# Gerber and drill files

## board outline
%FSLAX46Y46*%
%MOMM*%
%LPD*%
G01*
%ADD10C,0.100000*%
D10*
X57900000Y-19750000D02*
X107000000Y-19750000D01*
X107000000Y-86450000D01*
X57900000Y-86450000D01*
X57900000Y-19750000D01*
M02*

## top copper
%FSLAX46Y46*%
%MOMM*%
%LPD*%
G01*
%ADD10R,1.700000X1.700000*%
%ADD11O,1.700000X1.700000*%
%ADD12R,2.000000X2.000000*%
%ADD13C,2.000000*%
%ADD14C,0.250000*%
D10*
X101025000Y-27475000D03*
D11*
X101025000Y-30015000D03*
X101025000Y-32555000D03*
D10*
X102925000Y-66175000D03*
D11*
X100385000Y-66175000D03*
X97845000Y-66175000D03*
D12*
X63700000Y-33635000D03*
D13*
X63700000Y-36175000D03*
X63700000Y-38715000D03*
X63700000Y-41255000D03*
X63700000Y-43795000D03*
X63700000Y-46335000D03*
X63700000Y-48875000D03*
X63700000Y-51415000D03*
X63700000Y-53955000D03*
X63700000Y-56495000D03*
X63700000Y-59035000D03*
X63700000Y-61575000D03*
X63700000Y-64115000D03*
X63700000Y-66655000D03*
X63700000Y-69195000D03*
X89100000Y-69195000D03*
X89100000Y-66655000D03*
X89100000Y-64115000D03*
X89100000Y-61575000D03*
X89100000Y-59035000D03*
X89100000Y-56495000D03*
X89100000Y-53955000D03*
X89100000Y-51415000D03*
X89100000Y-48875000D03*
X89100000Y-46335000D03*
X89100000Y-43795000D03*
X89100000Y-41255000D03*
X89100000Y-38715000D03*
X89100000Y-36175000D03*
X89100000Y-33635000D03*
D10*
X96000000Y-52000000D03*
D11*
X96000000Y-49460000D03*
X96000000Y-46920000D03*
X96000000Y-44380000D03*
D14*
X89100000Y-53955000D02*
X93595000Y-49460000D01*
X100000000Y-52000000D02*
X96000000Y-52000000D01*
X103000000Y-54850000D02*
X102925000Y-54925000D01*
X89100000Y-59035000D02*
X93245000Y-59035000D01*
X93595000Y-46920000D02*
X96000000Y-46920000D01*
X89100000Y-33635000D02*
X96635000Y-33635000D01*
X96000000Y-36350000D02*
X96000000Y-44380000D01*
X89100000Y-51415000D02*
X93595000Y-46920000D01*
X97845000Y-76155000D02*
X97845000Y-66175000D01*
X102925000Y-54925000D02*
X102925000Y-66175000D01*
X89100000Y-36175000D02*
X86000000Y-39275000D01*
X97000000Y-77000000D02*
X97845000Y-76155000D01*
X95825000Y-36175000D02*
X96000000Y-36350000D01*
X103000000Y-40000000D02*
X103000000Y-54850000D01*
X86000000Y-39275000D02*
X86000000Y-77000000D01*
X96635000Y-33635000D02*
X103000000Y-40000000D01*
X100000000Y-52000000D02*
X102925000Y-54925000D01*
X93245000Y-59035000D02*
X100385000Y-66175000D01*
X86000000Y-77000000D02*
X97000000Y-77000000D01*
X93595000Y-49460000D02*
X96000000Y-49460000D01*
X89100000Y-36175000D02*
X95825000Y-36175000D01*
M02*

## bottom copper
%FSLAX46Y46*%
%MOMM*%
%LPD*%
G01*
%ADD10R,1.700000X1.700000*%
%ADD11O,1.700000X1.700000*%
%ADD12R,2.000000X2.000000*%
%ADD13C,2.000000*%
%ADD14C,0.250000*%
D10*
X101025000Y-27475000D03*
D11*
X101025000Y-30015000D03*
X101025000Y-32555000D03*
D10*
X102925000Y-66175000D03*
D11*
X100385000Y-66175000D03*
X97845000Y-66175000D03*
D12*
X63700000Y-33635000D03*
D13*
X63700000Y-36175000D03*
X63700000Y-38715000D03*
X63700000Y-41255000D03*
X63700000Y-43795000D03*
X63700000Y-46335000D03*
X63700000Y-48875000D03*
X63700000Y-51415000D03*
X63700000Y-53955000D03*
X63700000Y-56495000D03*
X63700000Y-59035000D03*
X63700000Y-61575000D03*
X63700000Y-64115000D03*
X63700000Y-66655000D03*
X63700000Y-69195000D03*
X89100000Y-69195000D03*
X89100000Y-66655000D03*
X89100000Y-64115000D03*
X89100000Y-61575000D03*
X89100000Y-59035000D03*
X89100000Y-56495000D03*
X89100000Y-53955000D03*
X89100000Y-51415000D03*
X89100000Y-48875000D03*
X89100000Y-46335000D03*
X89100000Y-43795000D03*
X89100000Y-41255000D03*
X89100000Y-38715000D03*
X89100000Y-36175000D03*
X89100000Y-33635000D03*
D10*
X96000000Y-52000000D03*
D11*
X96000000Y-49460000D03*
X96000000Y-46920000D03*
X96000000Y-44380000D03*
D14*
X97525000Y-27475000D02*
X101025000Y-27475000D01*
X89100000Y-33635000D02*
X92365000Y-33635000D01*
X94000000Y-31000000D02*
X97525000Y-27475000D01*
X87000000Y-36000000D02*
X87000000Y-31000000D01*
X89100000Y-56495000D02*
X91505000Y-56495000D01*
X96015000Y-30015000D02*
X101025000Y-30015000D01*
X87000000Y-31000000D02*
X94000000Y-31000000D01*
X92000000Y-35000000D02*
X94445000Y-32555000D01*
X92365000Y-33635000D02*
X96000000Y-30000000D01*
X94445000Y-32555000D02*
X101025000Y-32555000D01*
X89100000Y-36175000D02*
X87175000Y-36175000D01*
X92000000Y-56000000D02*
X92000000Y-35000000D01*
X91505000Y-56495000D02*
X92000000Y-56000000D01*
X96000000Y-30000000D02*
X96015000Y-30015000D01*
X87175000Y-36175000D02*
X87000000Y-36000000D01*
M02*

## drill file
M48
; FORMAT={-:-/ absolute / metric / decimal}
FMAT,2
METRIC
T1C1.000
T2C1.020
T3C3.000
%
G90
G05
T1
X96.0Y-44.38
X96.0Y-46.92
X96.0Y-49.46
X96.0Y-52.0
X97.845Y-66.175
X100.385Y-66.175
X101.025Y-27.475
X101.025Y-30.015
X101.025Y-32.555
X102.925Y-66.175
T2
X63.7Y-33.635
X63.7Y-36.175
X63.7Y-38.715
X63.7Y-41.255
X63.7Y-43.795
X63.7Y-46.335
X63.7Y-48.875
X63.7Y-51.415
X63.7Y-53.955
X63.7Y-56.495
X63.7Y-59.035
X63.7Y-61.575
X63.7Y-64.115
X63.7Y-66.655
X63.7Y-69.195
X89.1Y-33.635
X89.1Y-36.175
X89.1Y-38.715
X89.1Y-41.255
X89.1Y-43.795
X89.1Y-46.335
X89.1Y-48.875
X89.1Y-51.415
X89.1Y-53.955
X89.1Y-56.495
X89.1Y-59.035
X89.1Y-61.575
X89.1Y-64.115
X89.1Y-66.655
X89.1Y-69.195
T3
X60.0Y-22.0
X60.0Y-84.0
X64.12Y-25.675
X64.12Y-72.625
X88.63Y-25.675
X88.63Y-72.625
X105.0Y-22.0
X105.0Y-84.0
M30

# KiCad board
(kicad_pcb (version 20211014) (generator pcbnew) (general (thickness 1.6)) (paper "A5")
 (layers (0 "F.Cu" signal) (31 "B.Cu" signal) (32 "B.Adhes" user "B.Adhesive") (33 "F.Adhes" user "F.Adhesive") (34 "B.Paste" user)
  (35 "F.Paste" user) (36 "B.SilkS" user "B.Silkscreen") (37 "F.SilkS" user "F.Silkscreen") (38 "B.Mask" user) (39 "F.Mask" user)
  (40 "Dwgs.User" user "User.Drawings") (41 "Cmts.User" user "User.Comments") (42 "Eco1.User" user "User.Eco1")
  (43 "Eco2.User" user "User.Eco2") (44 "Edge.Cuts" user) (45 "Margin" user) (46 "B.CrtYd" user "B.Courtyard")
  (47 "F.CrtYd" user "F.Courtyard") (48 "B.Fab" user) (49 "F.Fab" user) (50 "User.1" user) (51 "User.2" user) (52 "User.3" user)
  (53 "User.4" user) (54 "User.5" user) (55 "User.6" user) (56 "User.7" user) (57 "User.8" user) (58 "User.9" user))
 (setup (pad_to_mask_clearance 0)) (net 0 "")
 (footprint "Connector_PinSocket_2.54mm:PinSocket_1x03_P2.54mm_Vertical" (layer "F.Cu") (at 101.025 27.475)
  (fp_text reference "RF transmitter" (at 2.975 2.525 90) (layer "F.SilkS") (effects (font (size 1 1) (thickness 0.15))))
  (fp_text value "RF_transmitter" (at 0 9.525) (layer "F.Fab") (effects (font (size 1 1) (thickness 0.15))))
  (pad "1" thru_hole rect (at 0 0) (size 1.7 1.7) (drill 1) (layers *.Cu *.Mask))
  (pad "2" thru_hole oval (at 0 2.54) (size 1.7 1.7) (drill 1) (layers *.Cu *.Mask))
  (pad "3" thru_hole oval (at 0 5.08) (size 1.7 1.7) (drill 1) (layers *.Cu *.Mask)))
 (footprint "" (layer "F.Cu") (at 105 22)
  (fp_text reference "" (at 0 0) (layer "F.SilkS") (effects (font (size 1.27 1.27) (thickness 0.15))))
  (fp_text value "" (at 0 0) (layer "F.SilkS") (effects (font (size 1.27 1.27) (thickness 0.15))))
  (pad "" np_thru_hole circle (at 0 0) (size 3 3) (drill 3) (layers *.Cu *.Mask)))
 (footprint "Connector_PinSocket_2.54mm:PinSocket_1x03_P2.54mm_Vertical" (layer "F.Cu") (at 102.925 66.175 -90)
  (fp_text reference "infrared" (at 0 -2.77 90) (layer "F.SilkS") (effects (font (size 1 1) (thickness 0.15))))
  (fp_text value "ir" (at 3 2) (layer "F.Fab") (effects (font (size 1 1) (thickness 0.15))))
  (pad "1" thru_hole rect (at 0 0 270) (size 1.7 1.7) (drill 1) (layers *.Cu *.Mask))
  (pad "2" thru_hole oval (at 0 2.54 270) (size 1.7 1.7) (drill 1) (layers *.Cu *.Mask))
  (pad "3" thru_hole oval (at 0 5.08 270) (size 1.7 1.7) (drill 1) (layers *.Cu *.Mask)))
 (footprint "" (layer "F.Cu") (at 105 84)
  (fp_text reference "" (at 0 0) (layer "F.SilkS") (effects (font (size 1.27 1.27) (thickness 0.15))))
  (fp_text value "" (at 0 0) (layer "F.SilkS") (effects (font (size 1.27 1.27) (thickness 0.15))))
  (pad "" np_thru_hole circle (at 0 0) (size 3 3) (drill 3) (layers *.Cu *.Mask)))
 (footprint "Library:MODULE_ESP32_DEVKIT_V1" (layer "F.Cu") (at 76.4 49.15)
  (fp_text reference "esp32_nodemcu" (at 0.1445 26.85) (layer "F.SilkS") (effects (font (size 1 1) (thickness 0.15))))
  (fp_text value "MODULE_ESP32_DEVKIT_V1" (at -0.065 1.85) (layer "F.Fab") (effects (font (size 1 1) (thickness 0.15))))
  (pad "" np_thru_hole circle (at -12.28 -23.475) (size 3 3) (drill 3) (layers *.Cu *.Mask))
  (pad "" np_thru_hole circle (at 12.23 23.475) (size 3 3) (drill 3) (layers *.Cu *.Mask))
  (pad "" np_thru_hole circle (at 12.23 -23.475) (size 3 3) (drill 3) (layers *.Cu *.Mask))
  (pad "" np_thru_hole circle (at -12.28 23.475) (size 3 3) (drill 3) (layers *.Cu *.Mask))
  (pad "1" thru_hole rect (at -12.7 -15.515) (size 2 2) (drill 1.02) (layers *.Cu *.Mask))
  (pad "2" thru_hole circle (at -12.7 -12.975) (size 2 2) (drill 1.02) (layers *.Cu *.Mask))
  (pad "3" thru_hole circle (at -12.7 -10.435) (size 2 2) (drill 1.02) (layers *.Cu *.Mask))
  (pad "4" thru_hole circle (at -12.7 -7.895) (size 2 2) (drill 1.02) (layers *.Cu *.Mask))
  (pad "5" thru_hole circle (at -12.7 -5.355) (size 2 2) (drill 1.02) (layers *.Cu *.Mask))
  (pad "6" thru_hole circle (at -12.7 -2.815) (size 2 2) (drill 1.02) (layers *.Cu *.Mask))
  (pad "7" thru_hole circle (at -12.7 -0.275) (size 2 2) (drill 1.02) (layers *.Cu *.Mask))
  (pad "8" thru_hole circle (at -12.7 2.265) (size 2 2) (drill 1.02) (layers *.Cu *.Mask))
  (pad "9" thru_hole circle (at -12.7 4.805) (size 2 2) (drill 1.02) (layers *.Cu *.Mask))
  (pad "10" thru_hole circle (at -12.7 7.345) (size 2 2) (drill 1.02) (layers *.Cu *.Mask))
  (pad "11" thru_hole circle (at -12.7 9.885) (size 2 2) (drill 1.02) (layers *.Cu *.Mask))
  (pad "12" thru_hole circle (at -12.7 12.425) (size 2 2) (drill 1.02) (layers *.Cu *.Mask))
  (pad "13" thru_hole circle (at -12.7 14.965) (size 2 2) (drill 1.02) (layers *.Cu *.Mask))
  (pad "14" thru_hole circle (at -12.7 17.505) (size 2 2) (drill 1.02) (layers *.Cu *.Mask))
  (pad "15" thru_hole circle (at -12.7 20.045) (size 2 2) (drill 1.02) (layers *.Cu *.Mask))
  (pad "16" thru_hole circle (at 12.7 20.045) (size 2 2) (drill 1.02) (layers *.Cu *.Mask))
  (pad "17" thru_hole circle (at 12.7 17.505) (size 2 2) (drill 1.02) (layers *.Cu *.Mask))
  (pad "18" thru_hole circle (at 12.7 14.965) (size 2 2) (drill 1.02) (layers *.Cu *.Mask))
  (pad "19" thru_hole circle (at 12.7 12.425) (size 2 2) (drill 1.02) (layers *.Cu *.Mask))
  (pad "20" thru_hole circle (at 12.7 9.885) (size 2 2) (drill 1.02) (layers *.Cu *.Mask))
  (pad "21" thru_hole circle (at 12.7 7.345) (size 2 2) (drill 1.02) (layers *.Cu *.Mask))
  (pad "22" thru_hole circle (at 12.7 4.805) (size 2 2) (drill 1.02) (layers *.Cu *.Mask))
  (pad "23" thru_hole circle (at 12.7 2.265) (size 2 2) (drill 1.02) (layers *.Cu *.Mask))
  (pad "24" thru_hole circle (at 12.7 -0.275) (size 2 2) (drill 1.02) (layers *.Cu *.Mask))
  (pad "25" thru_hole circle (at 12.7 -2.815) (size 2 2) (drill 1.02) (layers *.Cu *.Mask))
  (pad "26" thru_hole circle (at 12.7 -5.355) (size 2 2) (drill 1.02) (layers *.Cu *.Mask))
  (pad "27" thru_hole circle (at 12.7 -7.895) (size 2 2) (drill 1.02) (layers *.Cu *.Mask))
  (pad "28" thru_hole circle (at 12.7 -10.435) (size 2 2) (drill 1.02) (layers *.Cu *.Mask))
  (pad "29" thru_hole circle (at 12.7 -12.975) (size 2 2) (drill 1.02) (layers *.Cu *.Mask))
  (pad "30" thru_hole circle (at 12.7 -15.515) (size 2 2) (drill 1.02) (layers *.Cu *.Mask))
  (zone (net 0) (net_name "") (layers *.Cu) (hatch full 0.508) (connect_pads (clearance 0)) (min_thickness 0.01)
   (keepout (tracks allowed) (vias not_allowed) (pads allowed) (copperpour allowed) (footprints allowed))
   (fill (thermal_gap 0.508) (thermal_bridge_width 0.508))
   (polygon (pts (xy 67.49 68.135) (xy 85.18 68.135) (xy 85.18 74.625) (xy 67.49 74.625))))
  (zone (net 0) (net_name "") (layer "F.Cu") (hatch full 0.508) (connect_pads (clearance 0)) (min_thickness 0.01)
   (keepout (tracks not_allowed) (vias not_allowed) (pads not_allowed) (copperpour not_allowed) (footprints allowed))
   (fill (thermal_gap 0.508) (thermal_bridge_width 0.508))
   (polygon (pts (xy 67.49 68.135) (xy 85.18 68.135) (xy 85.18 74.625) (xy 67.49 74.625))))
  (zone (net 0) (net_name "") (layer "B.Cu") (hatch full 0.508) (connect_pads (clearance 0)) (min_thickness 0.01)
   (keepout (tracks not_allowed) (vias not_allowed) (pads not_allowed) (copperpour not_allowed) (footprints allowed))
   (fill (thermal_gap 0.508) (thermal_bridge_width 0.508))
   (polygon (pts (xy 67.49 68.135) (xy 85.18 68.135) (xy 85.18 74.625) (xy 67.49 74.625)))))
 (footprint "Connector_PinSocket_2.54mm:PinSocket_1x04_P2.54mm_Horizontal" (layer "F.Cu") (at 96 52 180)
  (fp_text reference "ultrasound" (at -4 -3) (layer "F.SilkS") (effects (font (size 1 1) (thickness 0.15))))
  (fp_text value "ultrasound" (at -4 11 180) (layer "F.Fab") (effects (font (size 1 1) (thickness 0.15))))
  (pad "1" thru_hole rect (at 0 0 180) (size 1.7 1.7) (drill 1) (layers *.Cu *.Mask))
  (pad "2" thru_hole oval (at 0 2.54 180) (size 1.7 1.7) (drill 1) (layers *.Cu *.Mask))
  (pad "3" thru_hole oval (at 0 5.08 180) (size 1.7 1.7) (drill 1) (layers *.Cu *.Mask))
  (pad "4" thru_hole oval (at 0 7.62 180) (size 1.7 1.7) (drill 1) (layers *.Cu *.Mask)))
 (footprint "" (layer "F.Cu") (at 60 22)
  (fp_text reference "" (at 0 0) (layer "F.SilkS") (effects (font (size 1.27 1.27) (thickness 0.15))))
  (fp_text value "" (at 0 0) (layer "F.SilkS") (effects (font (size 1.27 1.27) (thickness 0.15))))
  (pad "" np_thru_hole circle (at 0 0) (size 3 3) (drill 3) (layers *.Cu *.Mask)))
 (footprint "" (layer "F.Cu") (at 60 84)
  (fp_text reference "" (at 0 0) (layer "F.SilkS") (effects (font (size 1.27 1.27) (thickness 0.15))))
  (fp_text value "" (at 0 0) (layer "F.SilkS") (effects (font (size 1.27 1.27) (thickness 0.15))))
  (pad "" np_thru_hole circle (at 0 0) (size 3 3) (drill 3) (layers *.Cu *.Mask)))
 (gr_rect (start 107 19.75) (end 57.9 86.45) (layer "Edge.Cuts") (width 0.1) (fill none))
 (segment (start 89.1 53.955) (end 93.595 49.46) (width 0.25) (layer "F.Cu") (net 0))
 (segment (start 100 52) (end 96 52) (width 0.25) (layer "F.Cu") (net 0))
 (segment (start 103 54.85) (end 102.925 54.925) (width 0.25) (layer "F.Cu") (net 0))
 (segment (start 89.1 59.035) (end 93.245 59.035) (width 0.25) (layer "F.Cu") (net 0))
 (segment (start 93.595 46.92) (end 96 46.92) (width 0.25) (layer "F.Cu") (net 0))
 (segment (start 89.1 33.635) (end 96.635 33.635) (width 0.25) (layer "F.Cu") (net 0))
 (segment (start 96 36.35) (end 96 44.38) (width 0.25) (layer "F.Cu") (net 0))
 (segment (start 89.1 51.415) (end 93.595 46.92) (width 0.25) (layer "F.Cu") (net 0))
 (segment (start 97.845 76.155) (end 97.845 66.175) (width 0.25) (layer "F.Cu") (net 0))
 (segment (start 102.925 54.925) (end 102.925 66.175) (width 0.25) (layer "F.Cu") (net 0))
 (segment (start 89.1 36.175) (end 86 39.275) (width 0.25) (layer "F.Cu") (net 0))
 (segment (start 97 77) (end 97.845 76.155) (width 0.25) (layer "F.Cu") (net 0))
 (segment (start 95.825 36.175) (end 96 36.35) (width 0.25) (layer "F.Cu") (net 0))
 (segment (start 103 40) (end 103 54.85) (width 0.25) (layer "F.Cu") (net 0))
 (segment (start 86 39.275) (end 86 77) (width 0.25) (layer "F.Cu") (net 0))
 (segment (start 96.635 33.635) (end 103 40) (width 0.25) (layer "F.Cu") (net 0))
 (segment (start 100 52) (end 102.925 54.925) (width 0.25) (layer "F.Cu") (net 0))
 (segment (start 93.245 59.035) (end 100.385 66.175) (width 0.25) (layer "F.Cu") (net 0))
 (segment (start 86 77) (end 97 77) (width 0.25) (layer "F.Cu") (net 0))
 (segment (start 93.595 49.46) (end 96 49.46) (width 0.25) (layer "F.Cu") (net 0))
 (segment (start 89.1 36.175) (end 95.825 36.175) (width 0.25) (layer "F.Cu") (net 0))
 (segment (start 97.525 27.475) (end 101.025 27.475) (width 0.25) (layer "B.Cu") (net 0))
 (segment (start 89.1 33.635) (end 92.365 33.635) (width 0.25) (layer "B.Cu") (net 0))
 (segment (start 94 31) (end 97.525 27.475) (width 0.25) (layer "B.Cu") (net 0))
 (segment (start 87 36) (end 87 31) (width 0.25) (layer "B.Cu") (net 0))
 (segment (start 89.1 56.495) (end 91.505 56.495) (width 0.25) (layer "B.Cu") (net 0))
 (segment (start 96.015 30.015) (end 101.025 30.015) (width 0.25) (layer "B.Cu") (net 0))
 (segment (start 87 31) (end 94 31) (width 0.25) (layer "B.Cu") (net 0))
 (segment (start 92 35) (end 94.445 32.555) (width 0.25) (layer "B.Cu") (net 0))
 (segment (start 92.365 33.635) (end 96 30) (width 0.25) (layer "B.Cu") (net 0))
 (segment (start 94.445 32.555) (end 101.025 32.555) (width 0.25) (layer "B.Cu") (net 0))
 (segment (start 89.1 36.175) (end 87.175 36.175) (width 0.25) (layer "B.Cu") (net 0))
 (segment (start 92 56) (end 92 35) (width 0.25) (layer "B.Cu") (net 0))
 (segment (start 91.505 56.495) (end 92 56) (width 0.25) (layer "B.Cu") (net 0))
 (segment (start 96 30) (end 96.015 30.015) (width 0.25) (layer "B.Cu") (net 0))
 (segment (start 87.175 36.175) (end 87 36) (width 0.25) (layer "B.Cu") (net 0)))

